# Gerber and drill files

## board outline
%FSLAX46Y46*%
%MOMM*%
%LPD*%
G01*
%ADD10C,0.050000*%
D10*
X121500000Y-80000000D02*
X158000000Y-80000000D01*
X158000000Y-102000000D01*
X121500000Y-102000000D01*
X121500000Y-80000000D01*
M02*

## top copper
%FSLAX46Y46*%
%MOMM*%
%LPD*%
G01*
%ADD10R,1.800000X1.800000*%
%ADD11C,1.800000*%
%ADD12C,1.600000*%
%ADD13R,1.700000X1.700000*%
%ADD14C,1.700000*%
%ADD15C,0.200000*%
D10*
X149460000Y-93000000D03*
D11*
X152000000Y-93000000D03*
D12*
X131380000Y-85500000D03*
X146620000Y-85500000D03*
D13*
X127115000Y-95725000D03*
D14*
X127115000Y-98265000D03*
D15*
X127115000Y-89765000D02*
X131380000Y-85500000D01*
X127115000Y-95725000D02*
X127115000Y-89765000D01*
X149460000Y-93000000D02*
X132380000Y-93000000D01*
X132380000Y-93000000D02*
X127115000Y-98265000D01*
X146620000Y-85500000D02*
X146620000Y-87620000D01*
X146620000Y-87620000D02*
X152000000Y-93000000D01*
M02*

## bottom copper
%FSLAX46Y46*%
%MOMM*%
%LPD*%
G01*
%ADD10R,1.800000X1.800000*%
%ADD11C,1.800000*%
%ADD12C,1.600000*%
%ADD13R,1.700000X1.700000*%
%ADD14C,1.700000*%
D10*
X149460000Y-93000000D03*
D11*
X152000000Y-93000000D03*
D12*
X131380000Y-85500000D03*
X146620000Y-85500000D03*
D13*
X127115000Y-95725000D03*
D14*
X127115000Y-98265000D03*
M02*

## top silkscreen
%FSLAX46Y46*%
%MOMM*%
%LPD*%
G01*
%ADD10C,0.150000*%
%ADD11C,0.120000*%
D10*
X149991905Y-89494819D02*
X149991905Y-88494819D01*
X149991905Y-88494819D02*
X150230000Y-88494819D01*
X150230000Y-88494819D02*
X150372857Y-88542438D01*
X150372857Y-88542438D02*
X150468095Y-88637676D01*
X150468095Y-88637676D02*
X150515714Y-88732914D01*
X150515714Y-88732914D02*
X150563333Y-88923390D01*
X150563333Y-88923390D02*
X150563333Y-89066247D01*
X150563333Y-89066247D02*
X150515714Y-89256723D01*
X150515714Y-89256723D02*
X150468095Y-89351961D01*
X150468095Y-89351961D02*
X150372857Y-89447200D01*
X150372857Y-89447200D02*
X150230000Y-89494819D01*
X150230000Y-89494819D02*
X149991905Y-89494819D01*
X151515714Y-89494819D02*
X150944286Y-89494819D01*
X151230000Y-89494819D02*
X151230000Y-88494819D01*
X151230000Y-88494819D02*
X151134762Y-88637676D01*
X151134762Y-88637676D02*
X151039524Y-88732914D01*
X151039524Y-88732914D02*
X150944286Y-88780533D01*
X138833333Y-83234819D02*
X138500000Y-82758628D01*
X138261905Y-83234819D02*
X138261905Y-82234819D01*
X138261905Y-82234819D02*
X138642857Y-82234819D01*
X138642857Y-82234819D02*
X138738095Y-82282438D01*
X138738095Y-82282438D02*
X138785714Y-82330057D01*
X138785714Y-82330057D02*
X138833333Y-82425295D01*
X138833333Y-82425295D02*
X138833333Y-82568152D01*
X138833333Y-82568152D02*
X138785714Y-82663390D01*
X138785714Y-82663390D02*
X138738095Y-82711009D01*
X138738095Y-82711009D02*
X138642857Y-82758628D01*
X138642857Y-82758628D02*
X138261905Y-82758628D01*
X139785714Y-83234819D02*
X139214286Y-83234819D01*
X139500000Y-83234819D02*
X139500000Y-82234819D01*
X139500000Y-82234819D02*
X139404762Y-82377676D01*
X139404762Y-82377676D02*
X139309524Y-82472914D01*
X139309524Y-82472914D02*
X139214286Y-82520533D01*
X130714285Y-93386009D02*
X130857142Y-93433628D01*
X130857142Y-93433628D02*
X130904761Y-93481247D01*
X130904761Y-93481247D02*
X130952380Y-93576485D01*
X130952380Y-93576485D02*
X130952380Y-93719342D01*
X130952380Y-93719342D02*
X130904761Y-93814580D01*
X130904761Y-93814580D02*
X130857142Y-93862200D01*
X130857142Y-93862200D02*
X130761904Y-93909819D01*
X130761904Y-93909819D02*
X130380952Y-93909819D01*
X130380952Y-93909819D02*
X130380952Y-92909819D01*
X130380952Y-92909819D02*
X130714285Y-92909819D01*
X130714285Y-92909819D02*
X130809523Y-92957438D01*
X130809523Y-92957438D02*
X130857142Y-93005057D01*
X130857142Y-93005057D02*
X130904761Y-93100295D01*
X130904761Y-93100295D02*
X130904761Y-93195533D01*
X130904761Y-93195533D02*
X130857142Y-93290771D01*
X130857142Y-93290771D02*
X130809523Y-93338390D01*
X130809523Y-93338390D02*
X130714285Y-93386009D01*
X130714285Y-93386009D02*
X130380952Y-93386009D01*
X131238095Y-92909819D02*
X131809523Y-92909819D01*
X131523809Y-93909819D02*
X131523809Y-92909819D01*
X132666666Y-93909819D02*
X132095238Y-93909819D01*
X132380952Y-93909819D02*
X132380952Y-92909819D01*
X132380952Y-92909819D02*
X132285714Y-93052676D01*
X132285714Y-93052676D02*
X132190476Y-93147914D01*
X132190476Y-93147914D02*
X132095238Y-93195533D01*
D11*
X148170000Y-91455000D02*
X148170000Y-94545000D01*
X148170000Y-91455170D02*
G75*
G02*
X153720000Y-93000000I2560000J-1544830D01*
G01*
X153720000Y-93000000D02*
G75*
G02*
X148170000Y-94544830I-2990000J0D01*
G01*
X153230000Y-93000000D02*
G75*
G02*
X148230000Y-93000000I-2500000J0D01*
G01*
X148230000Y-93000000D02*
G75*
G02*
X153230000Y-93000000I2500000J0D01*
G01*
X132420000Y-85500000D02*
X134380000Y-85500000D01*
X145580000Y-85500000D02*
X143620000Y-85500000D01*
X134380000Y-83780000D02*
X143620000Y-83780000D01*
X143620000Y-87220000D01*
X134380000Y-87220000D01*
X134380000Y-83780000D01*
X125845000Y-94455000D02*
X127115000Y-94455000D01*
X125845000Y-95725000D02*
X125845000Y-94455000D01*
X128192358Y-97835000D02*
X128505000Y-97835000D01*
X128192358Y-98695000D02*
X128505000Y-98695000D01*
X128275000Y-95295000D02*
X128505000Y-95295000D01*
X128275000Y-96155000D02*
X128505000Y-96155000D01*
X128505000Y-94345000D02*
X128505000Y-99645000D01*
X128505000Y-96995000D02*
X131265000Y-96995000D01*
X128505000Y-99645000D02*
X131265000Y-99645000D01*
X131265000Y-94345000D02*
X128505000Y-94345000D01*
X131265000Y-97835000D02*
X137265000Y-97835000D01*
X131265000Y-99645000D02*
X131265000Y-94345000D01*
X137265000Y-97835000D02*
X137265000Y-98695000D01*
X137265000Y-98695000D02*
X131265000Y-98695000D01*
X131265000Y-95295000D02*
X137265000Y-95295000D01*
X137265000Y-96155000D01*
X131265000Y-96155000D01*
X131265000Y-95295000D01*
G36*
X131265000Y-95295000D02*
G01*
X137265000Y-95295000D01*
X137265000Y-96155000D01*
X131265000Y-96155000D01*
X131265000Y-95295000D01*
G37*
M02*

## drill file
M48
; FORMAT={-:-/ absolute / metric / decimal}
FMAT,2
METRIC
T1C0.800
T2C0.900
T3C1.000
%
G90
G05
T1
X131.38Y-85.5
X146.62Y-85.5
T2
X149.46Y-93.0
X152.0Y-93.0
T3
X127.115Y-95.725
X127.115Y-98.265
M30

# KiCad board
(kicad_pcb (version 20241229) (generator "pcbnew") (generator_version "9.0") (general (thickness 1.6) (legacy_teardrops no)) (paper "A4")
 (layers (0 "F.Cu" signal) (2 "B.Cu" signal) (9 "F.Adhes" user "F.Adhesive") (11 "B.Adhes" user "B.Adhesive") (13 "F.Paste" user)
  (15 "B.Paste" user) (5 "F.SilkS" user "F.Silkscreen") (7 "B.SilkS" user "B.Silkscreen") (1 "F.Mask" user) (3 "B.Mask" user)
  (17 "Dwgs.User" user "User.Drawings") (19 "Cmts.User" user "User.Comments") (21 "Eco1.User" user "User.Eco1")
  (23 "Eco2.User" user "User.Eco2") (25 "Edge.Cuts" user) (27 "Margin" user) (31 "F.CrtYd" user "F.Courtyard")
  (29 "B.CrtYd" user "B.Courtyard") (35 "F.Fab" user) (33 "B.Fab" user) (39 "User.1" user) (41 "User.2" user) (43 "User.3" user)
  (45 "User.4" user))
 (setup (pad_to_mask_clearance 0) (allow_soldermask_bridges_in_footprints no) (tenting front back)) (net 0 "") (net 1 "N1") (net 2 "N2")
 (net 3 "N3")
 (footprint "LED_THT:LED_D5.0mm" (layer "F.Cu") (at 149.46 93)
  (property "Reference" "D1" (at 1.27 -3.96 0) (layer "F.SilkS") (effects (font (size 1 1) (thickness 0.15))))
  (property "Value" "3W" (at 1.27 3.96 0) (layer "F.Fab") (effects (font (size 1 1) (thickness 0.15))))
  (fp_line (start -1.29 -1.545) (end -1.29 1.545) (stroke (width 0.12) (type solid)) (layer "F.SilkS"))
  (fp_arc (start -1.29 -1.54483) (mid 2.071779 -2.880495) (end 4.26 0) (stroke (width 0.12) (type solid)) (layer "F.SilkS"))
  (fp_arc (start 4.26 0) (mid 2.071779 2.880495) (end -1.29 1.54483) (stroke (width 0.12) (type solid)) (layer "F.SilkS"))
  (fp_circle (center 1.27 0) (end 3.77 0) (stroke (width 0.12) (type solid)) (fill no) (layer "F.SilkS"))
  (pad "1" thru_hole rect (at 0 0) (size 1.8 1.8) (drill 0.9) (layers "*.Cu" "*.Mask") (remove_unused_layers no) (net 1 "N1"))
  (pad "2" thru_hole circle (at 2.54 0) (size 1.8 1.8) (drill 0.9) (layers "*.Cu" "*.Mask") (remove_unused_layers no) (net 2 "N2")))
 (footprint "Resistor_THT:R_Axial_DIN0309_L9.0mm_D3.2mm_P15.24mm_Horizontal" (layer "F.Cu") (at 131.38 85.5)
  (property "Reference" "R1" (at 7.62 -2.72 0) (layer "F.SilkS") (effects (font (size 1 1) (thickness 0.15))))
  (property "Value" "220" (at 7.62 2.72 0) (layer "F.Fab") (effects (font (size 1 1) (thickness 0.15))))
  (fp_line (start 1.04 0) (end 3 0) (stroke (width 0.12) (type solid)) (layer "F.SilkS"))
  (fp_line (start 14.2 0) (end 12.24 0) (stroke (width 0.12) (type solid)) (layer "F.SilkS"))
  (fp_rect (start 3 -1.72) (end 12.24 1.72) (stroke (width 0.12) (type solid)) (fill no) (layer "F.SilkS"))
  (pad "1" thru_hole circle (at 0 0) (size 1.6 1.6) (drill 0.8) (layers "*.Cu" "*.Mask") (remove_unused_layers no) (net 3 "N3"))
  (pad "2" thru_hole circle (at 15.24 0) (size 1.6 1.6) (drill 0.8) (layers "*.Cu" "*.Mask") (remove_unused_layers no) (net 2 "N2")))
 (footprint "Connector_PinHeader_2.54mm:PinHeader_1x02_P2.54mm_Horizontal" (layer "F.Cu") (at 127.115 95.725)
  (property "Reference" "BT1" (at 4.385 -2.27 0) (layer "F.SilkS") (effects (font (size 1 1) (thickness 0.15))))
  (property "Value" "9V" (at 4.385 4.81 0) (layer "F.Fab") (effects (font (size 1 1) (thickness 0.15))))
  (fp_line (start -1.27 -1.27) (end 0 -1.27) (stroke (width 0.12) (type solid)) (layer "F.SilkS"))
  (fp_line (start -1.27 0) (end -1.27 -1.27) (stroke (width 0.12) (type solid)) (layer "F.SilkS"))
  (fp_line (start 1.077358 2.11) (end 1.39 2.11) (stroke (width 0.12) (type solid)) (layer "F.SilkS"))
  (fp_line (start 1.077358 2.97) (end 1.39 2.97) (stroke (width 0.12) (type solid)) (layer "F.SilkS"))
  (fp_line (start 1.16 -0.43) (end 1.39 -0.43) (stroke (width 0.12) (type solid)) (layer "F.SilkS"))
  (fp_line (start 1.16 0.43) (end 1.39 0.43) (stroke (width 0.12) (type solid)) (layer "F.SilkS"))
  (fp_line (start 1.39 -1.38) (end 1.39 3.92) (stroke (width 0.12) (type solid)) (layer "F.SilkS"))
  (fp_line (start 1.39 1.27) (end 4.15 1.27) (stroke (width 0.12) (type solid)) (layer "F.SilkS"))
  (fp_line (start 1.39 3.92) (end 4.15 3.92) (stroke (width 0.12) (type solid)) (layer "F.SilkS"))
  (fp_line (start 4.15 -1.38) (end 1.39 -1.38) (stroke (width 0.12) (type solid)) (layer "F.SilkS"))
  (fp_line (start 4.15 2.11) (end 10.15 2.11) (stroke (width 0.12) (type solid)) (layer "F.SilkS"))
  (fp_line (start 4.15 3.92) (end 4.15 -1.38) (stroke (width 0.12) (type solid)) (layer "F.SilkS"))
  (fp_line (start 10.15 2.11) (end 10.15 2.97) (stroke (width 0.12) (type solid)) (layer "F.SilkS"))
  (fp_line (start 10.15 2.97) (end 4.15 2.97) (stroke (width 0.12) (type solid)) (layer "F.SilkS"))
  (fp_rect (start 4.15 -0.43) (end 10.15 0.43) (stroke (width 0.12) (type solid)) (fill yes) (layer "F.SilkS"))
  (pad "1" thru_hole rect (at 0 0) (size 1.7 1.7) (drill 1) (layers "*.Cu" "*.Mask") (remove_unused_layers no) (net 3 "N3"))
  (pad "2" thru_hole circle (at 0 2.54) (size 1.7 1.7) (drill 1) (layers "*.Cu" "*.Mask") (remove_unused_layers no) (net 1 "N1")))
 (gr_rect (start 121.5 80) (end 158 102) (stroke (width 0.05) (type default)) (fill no) (layer "Edge.Cuts"))
 (segment (start 127.115 89.765) (end 131.38 85.5) (width 0.2) (layer "F.Cu") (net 3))
 (segment (start 127.115 95.725) (end 127.115 89.765) (width 0.2) (layer "F.Cu") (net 3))
 (segment (start 149.46 93) (end 132.38 93) (width 0.2) (layer "F.Cu") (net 1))
 (segment (start 132.38 93) (end 127.115 98.265) (width 0.2) (layer "F.Cu") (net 1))
 (segment (start 146.62 85.5) (end 146.62 87.62) (width 0.2) (layer "F.Cu") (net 2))
 (segment (start 146.62 87.62) (end 152 93) (width 0.2) (layer "F.Cu") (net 2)))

